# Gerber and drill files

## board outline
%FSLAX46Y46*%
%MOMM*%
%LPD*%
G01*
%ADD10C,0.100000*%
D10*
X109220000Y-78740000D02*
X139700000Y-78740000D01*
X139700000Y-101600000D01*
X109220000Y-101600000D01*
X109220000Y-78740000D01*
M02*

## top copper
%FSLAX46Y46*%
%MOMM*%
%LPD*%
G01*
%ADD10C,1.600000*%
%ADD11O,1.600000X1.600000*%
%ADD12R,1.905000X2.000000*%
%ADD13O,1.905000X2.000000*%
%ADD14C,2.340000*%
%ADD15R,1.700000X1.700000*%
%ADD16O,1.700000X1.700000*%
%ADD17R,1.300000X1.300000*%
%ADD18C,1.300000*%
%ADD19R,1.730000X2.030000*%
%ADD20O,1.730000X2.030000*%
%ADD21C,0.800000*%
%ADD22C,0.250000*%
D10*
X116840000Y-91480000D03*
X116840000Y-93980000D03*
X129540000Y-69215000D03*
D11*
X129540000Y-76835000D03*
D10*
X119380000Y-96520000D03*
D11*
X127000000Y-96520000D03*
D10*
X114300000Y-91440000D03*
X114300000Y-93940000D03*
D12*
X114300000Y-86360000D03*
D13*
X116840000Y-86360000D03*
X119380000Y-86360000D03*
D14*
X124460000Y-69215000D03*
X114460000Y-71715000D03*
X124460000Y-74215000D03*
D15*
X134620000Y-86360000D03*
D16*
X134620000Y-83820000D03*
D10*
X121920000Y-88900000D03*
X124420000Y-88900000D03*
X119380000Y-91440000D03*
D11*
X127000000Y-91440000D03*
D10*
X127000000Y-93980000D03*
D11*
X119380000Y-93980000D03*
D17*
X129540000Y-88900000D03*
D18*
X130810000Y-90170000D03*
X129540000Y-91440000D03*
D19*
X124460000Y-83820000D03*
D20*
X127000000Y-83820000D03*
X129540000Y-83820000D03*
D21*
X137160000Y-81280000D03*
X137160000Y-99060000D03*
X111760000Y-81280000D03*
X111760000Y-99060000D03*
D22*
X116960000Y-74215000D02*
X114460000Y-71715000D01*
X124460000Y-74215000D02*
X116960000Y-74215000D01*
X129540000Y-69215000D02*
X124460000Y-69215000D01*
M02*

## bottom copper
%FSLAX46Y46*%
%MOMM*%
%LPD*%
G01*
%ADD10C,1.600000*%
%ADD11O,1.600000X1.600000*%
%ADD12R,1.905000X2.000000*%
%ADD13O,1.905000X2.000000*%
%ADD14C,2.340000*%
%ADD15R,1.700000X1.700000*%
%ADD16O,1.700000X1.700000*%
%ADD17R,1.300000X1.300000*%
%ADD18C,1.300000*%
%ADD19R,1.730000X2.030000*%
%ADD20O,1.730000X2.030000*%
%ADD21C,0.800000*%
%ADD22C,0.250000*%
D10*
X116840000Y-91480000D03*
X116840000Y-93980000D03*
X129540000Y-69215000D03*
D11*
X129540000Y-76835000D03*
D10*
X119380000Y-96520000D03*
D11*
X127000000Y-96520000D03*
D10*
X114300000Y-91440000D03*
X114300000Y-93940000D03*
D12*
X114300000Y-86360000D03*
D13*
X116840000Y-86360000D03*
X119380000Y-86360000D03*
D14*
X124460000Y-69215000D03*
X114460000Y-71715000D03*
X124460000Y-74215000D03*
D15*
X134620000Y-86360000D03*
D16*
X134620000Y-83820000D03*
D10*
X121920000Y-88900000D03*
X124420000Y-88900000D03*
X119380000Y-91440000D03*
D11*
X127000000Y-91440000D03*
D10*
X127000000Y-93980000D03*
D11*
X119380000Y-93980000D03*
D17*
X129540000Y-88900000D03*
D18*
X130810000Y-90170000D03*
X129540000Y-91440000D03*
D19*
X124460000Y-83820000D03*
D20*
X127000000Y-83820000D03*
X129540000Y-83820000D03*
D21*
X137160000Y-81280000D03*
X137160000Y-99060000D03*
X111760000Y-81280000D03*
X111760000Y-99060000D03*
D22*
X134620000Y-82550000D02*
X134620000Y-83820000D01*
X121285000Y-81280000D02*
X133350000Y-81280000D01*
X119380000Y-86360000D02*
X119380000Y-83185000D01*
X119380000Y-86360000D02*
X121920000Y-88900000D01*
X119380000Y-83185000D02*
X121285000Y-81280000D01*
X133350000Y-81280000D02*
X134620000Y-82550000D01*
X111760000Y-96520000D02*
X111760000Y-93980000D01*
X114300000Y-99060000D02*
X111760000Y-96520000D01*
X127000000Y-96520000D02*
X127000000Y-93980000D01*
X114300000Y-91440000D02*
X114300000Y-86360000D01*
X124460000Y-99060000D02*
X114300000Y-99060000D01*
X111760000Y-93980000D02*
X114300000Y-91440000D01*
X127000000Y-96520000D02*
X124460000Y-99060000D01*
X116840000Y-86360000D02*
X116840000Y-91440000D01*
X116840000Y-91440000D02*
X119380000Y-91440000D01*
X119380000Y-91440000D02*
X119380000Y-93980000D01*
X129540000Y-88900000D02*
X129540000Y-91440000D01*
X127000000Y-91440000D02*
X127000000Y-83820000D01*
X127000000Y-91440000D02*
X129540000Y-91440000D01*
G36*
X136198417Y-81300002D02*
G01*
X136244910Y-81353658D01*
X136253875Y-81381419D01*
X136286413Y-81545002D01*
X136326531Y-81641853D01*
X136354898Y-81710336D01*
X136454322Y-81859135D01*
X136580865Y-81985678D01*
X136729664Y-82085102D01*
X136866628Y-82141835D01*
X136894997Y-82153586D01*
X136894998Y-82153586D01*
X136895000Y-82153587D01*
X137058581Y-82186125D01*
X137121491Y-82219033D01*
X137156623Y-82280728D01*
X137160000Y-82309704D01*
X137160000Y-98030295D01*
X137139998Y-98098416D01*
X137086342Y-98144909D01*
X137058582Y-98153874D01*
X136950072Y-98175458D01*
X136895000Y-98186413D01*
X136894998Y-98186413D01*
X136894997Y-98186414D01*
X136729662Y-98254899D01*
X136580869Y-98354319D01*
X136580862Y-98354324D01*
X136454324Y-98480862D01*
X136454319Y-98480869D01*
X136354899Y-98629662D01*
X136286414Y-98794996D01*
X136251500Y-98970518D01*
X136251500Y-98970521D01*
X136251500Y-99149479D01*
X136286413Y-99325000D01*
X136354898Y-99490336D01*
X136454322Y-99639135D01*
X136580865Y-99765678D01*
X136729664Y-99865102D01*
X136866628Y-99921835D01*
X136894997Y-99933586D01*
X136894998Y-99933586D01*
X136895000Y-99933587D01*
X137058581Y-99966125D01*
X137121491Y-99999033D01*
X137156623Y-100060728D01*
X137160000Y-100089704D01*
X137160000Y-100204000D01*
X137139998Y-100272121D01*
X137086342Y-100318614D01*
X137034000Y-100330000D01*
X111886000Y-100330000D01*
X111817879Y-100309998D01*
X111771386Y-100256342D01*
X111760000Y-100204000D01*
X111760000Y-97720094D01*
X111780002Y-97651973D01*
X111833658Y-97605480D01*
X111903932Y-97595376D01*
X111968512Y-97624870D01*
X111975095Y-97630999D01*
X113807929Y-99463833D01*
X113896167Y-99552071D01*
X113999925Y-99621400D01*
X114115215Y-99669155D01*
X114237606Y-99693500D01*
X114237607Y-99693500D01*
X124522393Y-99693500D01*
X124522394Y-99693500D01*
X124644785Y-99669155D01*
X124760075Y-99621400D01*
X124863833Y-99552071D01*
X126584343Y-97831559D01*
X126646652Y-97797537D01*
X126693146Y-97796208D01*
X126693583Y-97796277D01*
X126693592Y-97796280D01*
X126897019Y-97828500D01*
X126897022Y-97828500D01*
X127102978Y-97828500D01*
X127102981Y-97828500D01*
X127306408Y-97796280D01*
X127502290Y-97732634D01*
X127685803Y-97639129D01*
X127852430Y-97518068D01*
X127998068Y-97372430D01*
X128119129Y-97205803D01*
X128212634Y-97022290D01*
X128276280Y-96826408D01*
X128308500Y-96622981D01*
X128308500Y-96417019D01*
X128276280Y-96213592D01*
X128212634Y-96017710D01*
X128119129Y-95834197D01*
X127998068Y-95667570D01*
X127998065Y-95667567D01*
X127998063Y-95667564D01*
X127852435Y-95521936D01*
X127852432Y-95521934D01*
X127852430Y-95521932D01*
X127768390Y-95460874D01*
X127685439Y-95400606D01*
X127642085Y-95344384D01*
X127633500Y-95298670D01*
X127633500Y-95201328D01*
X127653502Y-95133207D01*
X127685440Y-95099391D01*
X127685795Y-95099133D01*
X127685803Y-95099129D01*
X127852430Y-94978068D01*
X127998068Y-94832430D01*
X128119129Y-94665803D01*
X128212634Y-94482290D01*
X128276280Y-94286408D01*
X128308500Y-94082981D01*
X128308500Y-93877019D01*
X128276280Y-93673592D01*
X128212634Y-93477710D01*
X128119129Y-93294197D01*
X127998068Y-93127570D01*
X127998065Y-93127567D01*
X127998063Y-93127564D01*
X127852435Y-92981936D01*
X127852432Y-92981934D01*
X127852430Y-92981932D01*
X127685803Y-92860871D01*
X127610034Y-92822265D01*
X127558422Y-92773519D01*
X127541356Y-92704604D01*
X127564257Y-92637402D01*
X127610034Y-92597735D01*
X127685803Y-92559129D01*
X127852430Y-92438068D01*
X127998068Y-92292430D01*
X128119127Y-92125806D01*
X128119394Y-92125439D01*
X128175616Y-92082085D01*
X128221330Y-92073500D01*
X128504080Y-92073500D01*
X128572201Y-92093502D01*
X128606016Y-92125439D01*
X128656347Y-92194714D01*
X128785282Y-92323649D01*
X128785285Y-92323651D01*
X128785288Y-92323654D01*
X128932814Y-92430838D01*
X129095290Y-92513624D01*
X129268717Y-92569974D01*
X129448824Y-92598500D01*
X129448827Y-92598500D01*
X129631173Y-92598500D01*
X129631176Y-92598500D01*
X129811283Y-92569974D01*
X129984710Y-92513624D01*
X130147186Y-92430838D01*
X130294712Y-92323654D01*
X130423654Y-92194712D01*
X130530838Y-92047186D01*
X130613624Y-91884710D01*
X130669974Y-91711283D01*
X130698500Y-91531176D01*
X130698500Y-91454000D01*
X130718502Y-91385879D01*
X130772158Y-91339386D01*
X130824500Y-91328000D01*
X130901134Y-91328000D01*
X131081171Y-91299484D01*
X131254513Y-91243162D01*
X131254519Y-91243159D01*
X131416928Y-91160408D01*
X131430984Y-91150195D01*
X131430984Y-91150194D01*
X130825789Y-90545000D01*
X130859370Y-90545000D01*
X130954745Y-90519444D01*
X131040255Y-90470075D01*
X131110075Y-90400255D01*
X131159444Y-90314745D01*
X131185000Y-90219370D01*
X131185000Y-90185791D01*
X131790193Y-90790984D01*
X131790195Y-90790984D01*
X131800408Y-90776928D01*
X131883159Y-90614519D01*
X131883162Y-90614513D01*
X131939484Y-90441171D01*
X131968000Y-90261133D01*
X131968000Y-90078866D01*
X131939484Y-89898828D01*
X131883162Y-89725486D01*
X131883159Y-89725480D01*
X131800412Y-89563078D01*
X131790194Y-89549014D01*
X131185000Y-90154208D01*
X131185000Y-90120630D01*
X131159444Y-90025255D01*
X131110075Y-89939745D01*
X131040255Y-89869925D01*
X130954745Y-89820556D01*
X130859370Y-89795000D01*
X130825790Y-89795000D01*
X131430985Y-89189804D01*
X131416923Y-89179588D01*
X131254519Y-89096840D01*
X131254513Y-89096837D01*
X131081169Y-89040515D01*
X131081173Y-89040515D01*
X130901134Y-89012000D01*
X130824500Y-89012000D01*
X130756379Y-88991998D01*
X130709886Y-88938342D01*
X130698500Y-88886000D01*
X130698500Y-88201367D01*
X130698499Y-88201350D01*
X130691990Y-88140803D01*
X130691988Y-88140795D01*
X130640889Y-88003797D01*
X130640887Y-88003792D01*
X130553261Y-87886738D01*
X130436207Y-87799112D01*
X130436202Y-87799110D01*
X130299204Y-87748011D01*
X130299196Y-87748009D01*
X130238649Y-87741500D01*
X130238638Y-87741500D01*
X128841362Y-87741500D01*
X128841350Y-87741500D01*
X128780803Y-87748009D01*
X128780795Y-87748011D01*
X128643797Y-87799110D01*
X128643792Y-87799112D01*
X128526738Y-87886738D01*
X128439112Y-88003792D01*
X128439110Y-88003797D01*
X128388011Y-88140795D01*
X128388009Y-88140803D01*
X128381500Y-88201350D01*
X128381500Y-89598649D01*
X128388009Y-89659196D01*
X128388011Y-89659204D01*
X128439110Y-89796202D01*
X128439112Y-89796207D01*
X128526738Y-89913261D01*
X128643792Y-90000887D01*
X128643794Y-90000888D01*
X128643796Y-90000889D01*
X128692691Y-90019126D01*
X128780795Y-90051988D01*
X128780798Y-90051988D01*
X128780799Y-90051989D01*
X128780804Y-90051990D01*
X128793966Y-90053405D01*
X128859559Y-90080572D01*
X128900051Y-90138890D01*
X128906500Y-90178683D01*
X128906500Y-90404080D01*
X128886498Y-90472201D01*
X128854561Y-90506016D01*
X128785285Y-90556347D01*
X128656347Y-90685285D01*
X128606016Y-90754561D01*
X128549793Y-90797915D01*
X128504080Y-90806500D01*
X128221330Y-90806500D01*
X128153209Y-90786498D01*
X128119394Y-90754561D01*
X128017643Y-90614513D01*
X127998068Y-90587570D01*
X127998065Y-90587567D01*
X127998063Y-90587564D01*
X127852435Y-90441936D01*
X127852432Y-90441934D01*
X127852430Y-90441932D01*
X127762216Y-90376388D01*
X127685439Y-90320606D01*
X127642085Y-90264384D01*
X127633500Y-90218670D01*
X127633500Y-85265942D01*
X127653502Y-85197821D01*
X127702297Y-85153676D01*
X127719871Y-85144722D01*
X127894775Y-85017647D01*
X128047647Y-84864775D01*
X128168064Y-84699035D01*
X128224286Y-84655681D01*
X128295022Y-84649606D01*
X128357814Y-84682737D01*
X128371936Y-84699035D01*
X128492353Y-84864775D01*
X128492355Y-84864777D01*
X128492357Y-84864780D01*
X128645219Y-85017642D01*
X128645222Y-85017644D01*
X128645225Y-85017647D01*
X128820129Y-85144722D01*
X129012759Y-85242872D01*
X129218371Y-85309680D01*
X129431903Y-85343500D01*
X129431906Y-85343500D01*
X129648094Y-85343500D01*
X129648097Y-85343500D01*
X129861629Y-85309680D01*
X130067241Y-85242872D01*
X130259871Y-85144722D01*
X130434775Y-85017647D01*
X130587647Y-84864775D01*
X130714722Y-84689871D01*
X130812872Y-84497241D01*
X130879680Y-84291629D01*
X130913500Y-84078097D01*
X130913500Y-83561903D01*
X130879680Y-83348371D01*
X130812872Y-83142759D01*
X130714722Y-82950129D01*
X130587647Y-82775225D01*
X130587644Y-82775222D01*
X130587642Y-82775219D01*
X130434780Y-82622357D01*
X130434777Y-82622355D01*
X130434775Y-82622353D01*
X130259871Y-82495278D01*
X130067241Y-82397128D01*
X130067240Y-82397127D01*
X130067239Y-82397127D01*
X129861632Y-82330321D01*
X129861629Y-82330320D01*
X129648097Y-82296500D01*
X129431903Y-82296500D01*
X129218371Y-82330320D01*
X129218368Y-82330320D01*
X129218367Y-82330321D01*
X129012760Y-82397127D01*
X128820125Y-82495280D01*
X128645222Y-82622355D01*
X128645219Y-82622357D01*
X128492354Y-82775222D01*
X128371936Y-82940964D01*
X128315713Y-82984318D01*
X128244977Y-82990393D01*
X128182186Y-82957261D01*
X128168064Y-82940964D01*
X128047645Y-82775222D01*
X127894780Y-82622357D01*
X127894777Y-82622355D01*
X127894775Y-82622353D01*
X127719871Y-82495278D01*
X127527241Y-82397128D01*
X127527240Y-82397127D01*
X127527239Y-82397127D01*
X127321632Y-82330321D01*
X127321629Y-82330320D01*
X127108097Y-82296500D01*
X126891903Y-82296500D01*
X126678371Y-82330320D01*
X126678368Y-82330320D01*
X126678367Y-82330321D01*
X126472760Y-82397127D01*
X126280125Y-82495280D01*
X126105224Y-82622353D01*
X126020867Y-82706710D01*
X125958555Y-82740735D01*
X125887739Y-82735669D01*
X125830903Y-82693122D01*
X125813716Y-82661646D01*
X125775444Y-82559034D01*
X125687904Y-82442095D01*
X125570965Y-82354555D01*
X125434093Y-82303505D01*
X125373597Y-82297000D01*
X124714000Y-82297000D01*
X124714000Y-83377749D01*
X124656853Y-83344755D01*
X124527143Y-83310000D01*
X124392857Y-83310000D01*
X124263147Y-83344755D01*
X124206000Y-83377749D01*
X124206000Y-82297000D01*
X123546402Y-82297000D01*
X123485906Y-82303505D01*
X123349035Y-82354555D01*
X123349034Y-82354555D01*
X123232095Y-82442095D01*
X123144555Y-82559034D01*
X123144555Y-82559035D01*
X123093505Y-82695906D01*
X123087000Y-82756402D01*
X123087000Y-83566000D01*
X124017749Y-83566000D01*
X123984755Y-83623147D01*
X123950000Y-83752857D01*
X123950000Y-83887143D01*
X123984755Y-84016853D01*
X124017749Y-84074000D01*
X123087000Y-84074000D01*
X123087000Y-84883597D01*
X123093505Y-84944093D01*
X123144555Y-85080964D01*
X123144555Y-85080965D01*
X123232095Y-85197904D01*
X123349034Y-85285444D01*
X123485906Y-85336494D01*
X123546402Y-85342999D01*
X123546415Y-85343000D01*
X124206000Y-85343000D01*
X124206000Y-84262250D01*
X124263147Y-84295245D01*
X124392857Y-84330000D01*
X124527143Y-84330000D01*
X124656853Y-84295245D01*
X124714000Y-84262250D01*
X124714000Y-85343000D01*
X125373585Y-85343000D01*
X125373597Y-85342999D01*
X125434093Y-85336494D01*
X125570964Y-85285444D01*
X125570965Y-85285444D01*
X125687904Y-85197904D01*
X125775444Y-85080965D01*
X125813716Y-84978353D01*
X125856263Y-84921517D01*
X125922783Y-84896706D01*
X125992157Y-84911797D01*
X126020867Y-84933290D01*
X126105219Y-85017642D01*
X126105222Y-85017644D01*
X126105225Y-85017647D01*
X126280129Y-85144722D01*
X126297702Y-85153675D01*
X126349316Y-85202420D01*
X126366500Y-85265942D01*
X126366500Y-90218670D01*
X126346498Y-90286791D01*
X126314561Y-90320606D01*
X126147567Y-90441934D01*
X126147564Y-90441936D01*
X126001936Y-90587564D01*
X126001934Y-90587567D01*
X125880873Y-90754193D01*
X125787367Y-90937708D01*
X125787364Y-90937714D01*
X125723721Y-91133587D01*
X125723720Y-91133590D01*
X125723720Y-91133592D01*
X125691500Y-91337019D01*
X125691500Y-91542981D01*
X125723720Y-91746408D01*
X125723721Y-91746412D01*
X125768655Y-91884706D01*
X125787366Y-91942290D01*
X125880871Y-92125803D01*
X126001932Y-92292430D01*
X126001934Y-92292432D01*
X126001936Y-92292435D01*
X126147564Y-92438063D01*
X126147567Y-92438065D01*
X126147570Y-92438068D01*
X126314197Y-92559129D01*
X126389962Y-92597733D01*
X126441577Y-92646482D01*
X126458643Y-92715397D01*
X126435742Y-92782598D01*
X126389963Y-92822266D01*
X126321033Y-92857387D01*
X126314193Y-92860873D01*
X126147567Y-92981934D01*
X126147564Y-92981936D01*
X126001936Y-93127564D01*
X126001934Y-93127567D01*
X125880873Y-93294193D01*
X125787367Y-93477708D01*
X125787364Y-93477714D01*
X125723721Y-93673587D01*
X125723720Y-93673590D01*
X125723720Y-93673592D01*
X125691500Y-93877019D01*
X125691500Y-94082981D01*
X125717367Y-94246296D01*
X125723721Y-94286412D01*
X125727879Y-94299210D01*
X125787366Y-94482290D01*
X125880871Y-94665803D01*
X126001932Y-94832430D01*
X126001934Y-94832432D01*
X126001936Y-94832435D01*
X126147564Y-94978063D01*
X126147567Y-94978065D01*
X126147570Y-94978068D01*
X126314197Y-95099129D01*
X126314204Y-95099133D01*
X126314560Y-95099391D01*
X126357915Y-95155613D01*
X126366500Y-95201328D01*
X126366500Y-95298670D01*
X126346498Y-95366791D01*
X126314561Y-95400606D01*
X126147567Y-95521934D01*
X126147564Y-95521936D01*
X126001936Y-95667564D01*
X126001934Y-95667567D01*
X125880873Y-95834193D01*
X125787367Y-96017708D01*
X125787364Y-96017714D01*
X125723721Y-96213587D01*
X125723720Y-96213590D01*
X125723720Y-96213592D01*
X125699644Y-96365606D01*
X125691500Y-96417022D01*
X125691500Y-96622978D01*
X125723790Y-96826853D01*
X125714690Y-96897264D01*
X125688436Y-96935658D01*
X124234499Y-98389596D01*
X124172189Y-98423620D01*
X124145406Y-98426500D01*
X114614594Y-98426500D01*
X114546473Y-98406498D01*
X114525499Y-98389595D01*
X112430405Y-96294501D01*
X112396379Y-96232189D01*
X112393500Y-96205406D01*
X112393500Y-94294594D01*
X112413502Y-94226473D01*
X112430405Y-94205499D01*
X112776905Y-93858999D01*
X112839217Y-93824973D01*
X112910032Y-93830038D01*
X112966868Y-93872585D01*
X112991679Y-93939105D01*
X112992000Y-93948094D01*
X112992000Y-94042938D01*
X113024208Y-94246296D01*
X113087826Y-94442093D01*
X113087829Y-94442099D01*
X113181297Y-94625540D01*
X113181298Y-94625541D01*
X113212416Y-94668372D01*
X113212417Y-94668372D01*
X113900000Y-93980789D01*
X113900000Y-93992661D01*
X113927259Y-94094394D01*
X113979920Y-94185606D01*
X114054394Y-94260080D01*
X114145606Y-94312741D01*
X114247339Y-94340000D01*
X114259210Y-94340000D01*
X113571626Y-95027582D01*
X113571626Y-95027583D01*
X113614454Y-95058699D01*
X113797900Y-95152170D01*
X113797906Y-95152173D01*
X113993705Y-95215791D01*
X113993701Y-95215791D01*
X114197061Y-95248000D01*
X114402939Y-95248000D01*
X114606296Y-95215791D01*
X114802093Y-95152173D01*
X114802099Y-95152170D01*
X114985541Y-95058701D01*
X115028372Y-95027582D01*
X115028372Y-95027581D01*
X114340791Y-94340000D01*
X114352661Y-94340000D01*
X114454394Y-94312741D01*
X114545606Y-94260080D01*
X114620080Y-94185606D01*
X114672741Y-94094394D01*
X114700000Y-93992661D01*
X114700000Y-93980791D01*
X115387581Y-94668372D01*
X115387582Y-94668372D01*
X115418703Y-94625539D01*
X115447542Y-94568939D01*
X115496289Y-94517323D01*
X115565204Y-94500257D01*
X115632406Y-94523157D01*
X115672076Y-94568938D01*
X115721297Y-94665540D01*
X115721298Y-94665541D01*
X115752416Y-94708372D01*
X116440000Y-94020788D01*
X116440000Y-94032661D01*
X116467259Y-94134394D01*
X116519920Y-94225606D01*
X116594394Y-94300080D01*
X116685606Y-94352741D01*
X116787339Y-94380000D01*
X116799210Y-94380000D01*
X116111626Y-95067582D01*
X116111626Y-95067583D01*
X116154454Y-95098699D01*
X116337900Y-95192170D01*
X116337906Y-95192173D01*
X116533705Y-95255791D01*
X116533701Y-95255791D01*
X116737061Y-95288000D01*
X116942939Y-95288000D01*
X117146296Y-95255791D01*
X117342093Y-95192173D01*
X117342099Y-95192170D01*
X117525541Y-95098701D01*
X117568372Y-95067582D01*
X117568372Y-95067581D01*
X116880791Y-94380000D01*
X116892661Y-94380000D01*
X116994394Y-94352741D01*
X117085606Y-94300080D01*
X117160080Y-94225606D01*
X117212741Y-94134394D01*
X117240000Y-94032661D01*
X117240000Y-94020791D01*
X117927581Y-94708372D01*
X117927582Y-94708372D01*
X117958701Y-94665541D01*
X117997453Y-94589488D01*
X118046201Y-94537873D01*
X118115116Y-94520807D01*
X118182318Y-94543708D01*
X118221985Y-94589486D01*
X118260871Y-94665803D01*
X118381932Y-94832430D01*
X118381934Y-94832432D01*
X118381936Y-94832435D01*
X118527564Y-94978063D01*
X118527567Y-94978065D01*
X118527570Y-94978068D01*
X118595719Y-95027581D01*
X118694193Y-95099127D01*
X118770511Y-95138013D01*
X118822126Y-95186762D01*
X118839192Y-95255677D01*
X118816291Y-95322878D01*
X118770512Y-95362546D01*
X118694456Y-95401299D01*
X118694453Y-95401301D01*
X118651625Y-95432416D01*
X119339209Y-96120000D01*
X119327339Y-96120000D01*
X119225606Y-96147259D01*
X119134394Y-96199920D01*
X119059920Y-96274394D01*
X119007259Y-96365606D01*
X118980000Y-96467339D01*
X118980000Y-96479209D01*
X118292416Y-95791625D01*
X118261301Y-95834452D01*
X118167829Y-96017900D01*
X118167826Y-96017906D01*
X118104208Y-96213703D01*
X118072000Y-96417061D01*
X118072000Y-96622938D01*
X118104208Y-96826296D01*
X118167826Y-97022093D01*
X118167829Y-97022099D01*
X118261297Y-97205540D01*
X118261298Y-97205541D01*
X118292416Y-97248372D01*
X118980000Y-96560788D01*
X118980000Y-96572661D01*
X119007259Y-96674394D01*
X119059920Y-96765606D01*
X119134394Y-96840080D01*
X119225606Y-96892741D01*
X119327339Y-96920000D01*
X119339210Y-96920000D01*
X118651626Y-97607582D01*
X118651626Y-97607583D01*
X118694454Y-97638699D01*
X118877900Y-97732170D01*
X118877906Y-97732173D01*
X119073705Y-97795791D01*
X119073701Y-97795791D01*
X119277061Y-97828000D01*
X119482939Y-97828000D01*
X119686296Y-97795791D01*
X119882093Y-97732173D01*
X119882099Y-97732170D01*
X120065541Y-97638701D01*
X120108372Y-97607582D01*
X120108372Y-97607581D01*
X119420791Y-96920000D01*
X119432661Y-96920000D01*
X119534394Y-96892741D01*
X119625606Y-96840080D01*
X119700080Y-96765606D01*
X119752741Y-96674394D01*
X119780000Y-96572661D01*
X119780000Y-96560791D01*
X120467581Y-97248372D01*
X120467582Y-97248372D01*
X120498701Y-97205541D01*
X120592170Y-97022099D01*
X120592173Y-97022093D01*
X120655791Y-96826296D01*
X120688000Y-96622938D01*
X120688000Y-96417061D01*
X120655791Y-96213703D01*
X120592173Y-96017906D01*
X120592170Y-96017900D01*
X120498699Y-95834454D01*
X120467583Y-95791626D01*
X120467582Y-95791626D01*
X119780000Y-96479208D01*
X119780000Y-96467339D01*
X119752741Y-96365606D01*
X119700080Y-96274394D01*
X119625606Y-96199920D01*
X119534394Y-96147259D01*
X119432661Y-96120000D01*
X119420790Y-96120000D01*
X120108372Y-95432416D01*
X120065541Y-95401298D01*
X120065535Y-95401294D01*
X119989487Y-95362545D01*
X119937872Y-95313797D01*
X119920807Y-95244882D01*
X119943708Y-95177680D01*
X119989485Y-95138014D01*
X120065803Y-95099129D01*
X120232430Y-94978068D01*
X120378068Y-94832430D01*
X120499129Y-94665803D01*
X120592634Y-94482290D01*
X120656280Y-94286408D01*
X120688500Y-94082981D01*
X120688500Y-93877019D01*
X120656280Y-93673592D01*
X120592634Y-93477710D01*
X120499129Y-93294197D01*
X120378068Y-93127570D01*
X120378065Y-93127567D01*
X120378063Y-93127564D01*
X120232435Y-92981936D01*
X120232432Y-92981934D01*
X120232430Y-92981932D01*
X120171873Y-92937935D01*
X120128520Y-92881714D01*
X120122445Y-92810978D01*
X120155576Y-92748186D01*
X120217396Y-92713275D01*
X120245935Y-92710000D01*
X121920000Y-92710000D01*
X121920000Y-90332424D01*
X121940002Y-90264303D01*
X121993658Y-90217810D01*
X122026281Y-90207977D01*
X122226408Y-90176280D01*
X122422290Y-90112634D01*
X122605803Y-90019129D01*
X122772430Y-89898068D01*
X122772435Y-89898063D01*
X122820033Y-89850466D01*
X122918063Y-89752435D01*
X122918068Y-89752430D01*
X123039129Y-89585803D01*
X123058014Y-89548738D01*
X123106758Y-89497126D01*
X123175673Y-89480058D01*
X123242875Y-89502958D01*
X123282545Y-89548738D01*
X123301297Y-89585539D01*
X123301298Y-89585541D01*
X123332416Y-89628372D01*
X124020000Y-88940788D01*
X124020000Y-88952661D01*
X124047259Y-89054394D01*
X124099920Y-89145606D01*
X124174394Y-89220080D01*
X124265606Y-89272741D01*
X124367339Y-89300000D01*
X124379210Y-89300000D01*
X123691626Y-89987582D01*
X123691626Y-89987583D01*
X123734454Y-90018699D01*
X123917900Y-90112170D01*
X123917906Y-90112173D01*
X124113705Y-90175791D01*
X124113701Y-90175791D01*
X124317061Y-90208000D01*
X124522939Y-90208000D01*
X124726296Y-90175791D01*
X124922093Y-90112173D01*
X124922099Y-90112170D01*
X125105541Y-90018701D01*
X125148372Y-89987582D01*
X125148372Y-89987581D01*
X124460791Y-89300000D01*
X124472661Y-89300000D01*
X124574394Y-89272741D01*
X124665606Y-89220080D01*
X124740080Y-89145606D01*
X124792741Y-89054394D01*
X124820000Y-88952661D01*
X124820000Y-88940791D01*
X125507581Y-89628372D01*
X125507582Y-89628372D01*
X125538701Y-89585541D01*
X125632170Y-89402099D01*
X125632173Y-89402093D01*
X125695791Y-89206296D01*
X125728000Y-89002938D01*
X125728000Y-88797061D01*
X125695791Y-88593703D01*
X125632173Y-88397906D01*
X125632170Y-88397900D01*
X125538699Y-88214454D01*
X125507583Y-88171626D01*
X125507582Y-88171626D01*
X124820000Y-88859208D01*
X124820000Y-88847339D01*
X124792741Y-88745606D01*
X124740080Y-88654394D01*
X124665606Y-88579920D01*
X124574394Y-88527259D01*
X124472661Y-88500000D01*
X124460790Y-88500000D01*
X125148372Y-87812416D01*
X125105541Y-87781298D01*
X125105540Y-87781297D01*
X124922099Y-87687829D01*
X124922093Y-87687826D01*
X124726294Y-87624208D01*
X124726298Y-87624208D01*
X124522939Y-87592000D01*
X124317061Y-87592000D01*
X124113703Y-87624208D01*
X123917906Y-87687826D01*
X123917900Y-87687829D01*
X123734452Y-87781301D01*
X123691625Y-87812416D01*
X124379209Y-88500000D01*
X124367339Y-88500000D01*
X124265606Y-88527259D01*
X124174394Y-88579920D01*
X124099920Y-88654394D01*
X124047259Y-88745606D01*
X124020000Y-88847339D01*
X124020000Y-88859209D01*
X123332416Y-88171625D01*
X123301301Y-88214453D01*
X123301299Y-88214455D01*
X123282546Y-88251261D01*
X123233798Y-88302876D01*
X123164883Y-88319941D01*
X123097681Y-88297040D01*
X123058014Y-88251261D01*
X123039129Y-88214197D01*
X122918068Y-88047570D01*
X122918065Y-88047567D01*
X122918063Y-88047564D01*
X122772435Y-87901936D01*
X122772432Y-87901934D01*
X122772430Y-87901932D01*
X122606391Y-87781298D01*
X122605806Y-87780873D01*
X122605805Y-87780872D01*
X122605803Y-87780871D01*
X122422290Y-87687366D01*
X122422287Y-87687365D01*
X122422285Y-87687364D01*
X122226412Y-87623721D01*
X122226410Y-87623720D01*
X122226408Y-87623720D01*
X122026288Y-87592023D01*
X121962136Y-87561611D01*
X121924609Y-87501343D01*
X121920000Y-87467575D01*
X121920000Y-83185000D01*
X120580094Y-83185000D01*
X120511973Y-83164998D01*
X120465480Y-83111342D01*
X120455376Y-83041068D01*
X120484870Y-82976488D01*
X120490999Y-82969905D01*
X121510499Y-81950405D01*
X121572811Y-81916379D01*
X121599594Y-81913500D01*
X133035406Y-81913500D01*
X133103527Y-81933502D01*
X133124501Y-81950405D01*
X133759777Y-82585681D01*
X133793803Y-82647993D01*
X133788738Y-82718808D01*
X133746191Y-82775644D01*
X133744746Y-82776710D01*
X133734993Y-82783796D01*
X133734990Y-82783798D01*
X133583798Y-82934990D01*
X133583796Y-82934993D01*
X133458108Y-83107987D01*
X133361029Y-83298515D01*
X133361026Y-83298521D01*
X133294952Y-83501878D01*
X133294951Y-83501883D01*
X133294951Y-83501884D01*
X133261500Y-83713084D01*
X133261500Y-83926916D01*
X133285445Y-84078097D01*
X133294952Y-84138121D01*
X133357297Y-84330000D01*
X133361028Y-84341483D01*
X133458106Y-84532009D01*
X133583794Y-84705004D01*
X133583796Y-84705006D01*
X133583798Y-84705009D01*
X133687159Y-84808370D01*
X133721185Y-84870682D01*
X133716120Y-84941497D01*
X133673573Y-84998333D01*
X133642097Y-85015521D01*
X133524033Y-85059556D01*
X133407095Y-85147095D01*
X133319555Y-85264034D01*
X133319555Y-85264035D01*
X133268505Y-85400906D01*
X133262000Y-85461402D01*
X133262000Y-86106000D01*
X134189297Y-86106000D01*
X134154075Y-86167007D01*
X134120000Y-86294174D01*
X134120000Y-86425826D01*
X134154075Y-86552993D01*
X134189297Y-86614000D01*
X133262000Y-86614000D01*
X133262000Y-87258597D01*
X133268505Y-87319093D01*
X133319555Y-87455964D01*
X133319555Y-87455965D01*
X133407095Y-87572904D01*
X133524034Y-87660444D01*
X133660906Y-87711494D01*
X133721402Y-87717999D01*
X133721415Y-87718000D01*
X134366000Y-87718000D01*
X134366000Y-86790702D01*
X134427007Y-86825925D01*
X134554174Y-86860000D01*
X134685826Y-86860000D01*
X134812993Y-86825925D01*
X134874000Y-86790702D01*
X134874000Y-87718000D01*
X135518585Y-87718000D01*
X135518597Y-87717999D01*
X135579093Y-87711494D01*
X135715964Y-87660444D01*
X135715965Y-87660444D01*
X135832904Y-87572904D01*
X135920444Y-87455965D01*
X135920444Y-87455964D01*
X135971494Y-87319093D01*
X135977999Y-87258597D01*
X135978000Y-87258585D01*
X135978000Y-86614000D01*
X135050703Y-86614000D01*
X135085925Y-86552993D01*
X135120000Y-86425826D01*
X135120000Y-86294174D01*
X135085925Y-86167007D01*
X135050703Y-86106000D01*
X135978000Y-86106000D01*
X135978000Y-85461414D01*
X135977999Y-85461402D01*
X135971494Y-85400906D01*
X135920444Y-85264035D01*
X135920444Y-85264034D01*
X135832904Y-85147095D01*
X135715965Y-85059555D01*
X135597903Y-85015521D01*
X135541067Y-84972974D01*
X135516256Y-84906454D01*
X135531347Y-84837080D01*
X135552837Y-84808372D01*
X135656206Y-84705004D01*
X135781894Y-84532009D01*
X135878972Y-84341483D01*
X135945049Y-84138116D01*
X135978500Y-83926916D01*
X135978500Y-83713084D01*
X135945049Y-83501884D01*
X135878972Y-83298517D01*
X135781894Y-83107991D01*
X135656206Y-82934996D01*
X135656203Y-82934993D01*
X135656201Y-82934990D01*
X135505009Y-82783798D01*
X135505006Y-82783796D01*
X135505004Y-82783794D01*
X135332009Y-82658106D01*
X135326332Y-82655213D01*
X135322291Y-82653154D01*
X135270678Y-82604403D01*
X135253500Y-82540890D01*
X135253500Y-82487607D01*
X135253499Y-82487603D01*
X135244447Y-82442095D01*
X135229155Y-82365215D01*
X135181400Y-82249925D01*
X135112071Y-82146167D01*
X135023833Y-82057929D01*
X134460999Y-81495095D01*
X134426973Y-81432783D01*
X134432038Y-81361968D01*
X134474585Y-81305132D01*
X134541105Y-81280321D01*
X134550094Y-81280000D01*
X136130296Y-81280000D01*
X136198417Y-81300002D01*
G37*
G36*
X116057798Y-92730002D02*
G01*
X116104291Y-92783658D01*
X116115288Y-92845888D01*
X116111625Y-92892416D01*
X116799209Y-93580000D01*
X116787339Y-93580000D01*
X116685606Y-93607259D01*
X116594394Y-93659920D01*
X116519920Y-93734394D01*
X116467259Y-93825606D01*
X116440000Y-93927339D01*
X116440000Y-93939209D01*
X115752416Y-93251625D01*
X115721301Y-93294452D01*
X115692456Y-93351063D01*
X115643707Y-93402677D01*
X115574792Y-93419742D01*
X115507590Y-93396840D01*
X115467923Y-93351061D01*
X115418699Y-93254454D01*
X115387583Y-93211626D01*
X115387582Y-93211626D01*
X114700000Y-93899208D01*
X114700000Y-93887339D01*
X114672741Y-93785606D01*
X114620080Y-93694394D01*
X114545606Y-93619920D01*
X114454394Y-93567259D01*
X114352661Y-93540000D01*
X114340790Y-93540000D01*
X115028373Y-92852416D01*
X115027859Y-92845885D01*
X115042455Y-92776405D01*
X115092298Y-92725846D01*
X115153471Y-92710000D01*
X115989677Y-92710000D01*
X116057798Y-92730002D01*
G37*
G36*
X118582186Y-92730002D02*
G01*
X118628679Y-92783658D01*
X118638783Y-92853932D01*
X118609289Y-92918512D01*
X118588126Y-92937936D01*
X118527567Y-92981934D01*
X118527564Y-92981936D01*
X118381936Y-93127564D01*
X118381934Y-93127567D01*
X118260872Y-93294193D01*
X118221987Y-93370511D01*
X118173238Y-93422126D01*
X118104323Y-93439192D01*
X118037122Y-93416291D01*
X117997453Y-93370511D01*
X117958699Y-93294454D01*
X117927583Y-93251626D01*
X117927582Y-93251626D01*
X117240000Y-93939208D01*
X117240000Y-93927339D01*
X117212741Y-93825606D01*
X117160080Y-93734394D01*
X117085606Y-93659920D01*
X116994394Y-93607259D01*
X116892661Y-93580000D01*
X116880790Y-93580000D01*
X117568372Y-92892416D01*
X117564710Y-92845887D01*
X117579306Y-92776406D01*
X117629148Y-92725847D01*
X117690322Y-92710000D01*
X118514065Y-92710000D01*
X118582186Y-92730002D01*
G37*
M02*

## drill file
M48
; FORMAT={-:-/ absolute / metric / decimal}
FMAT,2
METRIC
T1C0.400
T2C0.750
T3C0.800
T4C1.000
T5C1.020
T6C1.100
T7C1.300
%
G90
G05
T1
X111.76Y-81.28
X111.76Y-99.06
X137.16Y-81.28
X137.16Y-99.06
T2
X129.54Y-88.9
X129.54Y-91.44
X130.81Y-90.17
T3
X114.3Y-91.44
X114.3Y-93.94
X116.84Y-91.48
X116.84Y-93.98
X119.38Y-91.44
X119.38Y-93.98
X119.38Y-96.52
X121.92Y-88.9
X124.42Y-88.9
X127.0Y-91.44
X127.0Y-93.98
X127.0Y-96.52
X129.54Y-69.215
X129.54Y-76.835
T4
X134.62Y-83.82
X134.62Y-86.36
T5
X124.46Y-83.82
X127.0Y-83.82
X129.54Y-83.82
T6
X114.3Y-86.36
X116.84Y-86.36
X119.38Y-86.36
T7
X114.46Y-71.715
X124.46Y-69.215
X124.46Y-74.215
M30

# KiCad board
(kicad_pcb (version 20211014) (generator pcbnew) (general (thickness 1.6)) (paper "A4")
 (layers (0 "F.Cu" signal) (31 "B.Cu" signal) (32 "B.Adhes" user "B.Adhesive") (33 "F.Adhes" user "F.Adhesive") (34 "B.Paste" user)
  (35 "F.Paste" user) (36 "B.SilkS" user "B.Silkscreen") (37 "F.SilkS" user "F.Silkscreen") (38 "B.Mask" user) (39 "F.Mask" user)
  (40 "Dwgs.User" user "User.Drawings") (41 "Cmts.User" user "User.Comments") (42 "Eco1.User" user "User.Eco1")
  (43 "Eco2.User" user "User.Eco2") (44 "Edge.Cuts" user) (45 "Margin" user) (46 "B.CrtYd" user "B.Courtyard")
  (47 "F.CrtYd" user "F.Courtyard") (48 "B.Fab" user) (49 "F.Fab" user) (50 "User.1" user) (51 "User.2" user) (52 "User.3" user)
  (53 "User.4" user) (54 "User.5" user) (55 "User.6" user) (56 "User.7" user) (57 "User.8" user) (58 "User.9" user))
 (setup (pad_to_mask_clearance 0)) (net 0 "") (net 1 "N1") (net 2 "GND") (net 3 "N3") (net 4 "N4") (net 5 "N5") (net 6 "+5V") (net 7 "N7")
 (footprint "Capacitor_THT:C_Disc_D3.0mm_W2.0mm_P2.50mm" (layer "F.Cu") (at 116.84 91.48 -90)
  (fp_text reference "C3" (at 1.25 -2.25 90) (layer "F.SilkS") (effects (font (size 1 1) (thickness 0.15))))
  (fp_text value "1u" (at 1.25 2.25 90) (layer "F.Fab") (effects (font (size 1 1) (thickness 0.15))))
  (pad "1" thru_hole circle (at 0 0 270) (size 1.6 1.6) (drill 0.8) (layers *.Cu *.Mask) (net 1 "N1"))
  (pad "2" thru_hole circle (at 2.5 0 270) (size 1.6 1.6) (drill 0.8) (layers *.Cu *.Mask) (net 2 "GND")))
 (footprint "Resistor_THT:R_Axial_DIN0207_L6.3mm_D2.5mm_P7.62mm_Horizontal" (layer "F.Cu") (at 129.54 69.215 -90)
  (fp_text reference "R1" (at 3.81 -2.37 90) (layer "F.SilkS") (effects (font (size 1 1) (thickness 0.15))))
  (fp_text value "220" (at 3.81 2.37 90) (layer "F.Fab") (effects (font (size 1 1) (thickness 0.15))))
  (pad "1" thru_hole circle (at 0 0 270) (size 1.6 1.6) (drill 0.8) (layers *.Cu *.Mask) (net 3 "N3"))
  (pad "2" thru_hole oval (at 7.62 0 270) (size 1.6 1.6) (drill 0.8) (layers *.Cu *.Mask) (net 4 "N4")))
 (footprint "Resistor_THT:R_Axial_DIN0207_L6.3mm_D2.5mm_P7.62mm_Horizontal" (layer "F.Cu") (at 119.38 96.52)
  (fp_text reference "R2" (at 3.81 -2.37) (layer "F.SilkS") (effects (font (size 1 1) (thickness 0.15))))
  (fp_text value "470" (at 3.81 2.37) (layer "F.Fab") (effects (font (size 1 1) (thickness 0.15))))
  (pad "1" thru_hole circle (at 0 0) (size 1.6 1.6) (drill 0.8) (layers *.Cu *.Mask) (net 2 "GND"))
  (pad "2" thru_hole oval (at 7.62 0) (size 1.6 1.6) (drill 0.8) (layers *.Cu *.Mask) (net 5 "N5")))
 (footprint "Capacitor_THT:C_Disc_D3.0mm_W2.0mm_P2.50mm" (layer "F.Cu") (at 114.3 91.44 -90)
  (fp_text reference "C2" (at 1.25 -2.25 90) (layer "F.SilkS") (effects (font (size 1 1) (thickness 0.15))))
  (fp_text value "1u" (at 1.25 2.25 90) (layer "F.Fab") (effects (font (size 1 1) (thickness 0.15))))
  (pad "1" thru_hole circle (at 0 0 270) (size 1.6 1.6) (drill 0.8) (layers *.Cu *.Mask) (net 5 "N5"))
  (pad "2" thru_hole circle (at 2.5 0 270) (size 1.6 1.6) (drill 0.8) (layers *.Cu *.Mask) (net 2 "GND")))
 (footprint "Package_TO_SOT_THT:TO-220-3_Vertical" (layer "F.Cu") (at 114.3 86.36) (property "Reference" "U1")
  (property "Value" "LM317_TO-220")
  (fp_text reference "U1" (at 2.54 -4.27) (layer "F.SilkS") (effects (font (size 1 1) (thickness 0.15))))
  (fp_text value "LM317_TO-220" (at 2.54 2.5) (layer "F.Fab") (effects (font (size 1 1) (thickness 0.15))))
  (pad "1" thru_hole rect (at 0 0) (size 1.905 2) (drill 1.1) (layers *.Cu *.Mask) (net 5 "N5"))
  (pad "2" thru_hole oval (at 2.54 0) (size 1.905 2) (drill 1.1) (layers *.Cu *.Mask) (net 1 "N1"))
  (pad "3" thru_hole oval (at 5.08 0) (size 1.905 2) (drill 1.1) (layers *.Cu *.Mask) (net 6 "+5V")))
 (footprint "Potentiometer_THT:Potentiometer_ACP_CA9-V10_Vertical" (layer "F.Cu") (at 124.46 69.215 180) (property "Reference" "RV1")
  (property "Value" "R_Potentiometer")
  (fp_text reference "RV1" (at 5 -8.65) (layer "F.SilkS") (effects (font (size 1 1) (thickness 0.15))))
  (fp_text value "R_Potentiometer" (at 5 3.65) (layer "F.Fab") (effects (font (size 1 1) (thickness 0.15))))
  (pad "1" thru_hole circle (at 0 0 180) (size 2.34 2.34) (drill 1.3) (layers *.Cu *.Mask) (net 3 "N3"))
  (pad "2" thru_hole circle (at 10 -2.5 180) (size 2.34 2.34) (drill 1.3) (layers *.Cu *.Mask) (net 2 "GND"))
  (pad "3" thru_hole circle (at 0 -5 180) (size 2.34 2.34) (drill 1.3) (layers *.Cu *.Mask) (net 2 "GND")))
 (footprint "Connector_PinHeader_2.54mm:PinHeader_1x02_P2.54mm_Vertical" (layer "F.Cu") (at 134.62 86.36 180) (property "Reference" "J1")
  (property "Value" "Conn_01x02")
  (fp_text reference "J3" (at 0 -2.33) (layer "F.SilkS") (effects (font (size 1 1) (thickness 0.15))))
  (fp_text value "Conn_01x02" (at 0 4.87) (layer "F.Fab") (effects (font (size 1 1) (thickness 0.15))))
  (pad "1" thru_hole rect (at 0 0 180) (size 1.7 1.7) (drill 1) (layers *.Cu *.Mask) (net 2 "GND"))
  (pad "2" thru_hole oval (at 0 2.54 180) (size 1.7 1.7) (drill 1) (layers *.Cu *.Mask) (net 6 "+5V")))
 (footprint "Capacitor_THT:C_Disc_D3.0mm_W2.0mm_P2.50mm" (layer "F.Cu") (at 121.92 88.9) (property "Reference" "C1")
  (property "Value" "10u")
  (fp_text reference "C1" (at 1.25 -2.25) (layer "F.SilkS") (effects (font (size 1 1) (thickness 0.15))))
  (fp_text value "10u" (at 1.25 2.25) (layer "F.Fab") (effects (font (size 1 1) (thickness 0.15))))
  (pad "1" thru_hole circle (at 0 0) (size 1.6 1.6) (drill 0.8) (layers *.Cu *.Mask) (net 6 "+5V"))
  (pad "2" thru_hole circle (at 2.5 0) (size 1.6 1.6) (drill 0.8) (layers *.Cu *.Mask) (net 2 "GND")))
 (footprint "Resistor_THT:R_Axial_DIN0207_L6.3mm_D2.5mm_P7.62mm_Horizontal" (layer "F.Cu") (at 119.38 91.44)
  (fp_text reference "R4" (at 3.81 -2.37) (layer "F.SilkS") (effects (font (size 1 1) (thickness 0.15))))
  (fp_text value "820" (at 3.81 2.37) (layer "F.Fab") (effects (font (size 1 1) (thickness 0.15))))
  (pad "1" thru_hole circle (at 0 0) (size 1.6 1.6) (drill 0.8) (layers *.Cu *.Mask) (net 1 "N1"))
  (pad "2" thru_hole oval (at 7.62 0) (size 1.6 1.6) (drill 0.8) (layers *.Cu *.Mask) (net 4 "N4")))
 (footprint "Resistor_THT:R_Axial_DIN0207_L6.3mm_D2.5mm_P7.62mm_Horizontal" (layer "F.Cu") (at 127 93.98 180) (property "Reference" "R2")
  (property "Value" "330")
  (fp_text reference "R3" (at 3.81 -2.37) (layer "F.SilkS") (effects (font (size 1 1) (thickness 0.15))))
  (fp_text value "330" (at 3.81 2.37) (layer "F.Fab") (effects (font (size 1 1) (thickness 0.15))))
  (pad "1" thru_hole circle (at 0 0 180) (size 1.6 1.6) (drill 0.8) (layers *.Cu *.Mask) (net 5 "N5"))
  (pad "2" thru_hole oval (at 7.62 0 180) (size 1.6 1.6) (drill 0.8) (layers *.Cu *.Mask) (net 1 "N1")))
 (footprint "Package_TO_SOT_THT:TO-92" (layer "F.Cu") (at 129.54 88.9 -90) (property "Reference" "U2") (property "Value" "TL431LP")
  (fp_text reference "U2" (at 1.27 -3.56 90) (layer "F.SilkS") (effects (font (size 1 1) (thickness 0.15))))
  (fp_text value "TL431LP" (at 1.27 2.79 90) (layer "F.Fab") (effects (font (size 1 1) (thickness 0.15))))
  (pad "1" thru_hole rect (at 0 0 270) (size 1.3 1.3) (drill 0.75) (layers *.Cu *.Mask) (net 4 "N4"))
  (pad "2" thru_hole circle (at 1.27 -1.27 270) (size 1.3 1.3) (drill 0.75) (layers *.Cu *.Mask) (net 2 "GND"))
  (pad "3" thru_hole circle (at 2.54 0 270) (size 1.3 1.3) (drill 0.75) (layers *.Cu *.Mask) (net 4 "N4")))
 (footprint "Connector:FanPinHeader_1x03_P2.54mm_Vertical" (layer "F.Cu") (at 124.46 83.82) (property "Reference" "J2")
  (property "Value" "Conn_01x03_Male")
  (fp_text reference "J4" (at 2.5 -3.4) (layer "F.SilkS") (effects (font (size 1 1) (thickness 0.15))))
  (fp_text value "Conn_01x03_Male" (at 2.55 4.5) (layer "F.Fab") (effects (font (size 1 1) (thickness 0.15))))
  (pad "1" thru_hole rect (at 0 0 90) (size 2.03 1.73) (drill 1.02) (layers *.Cu *.Mask) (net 2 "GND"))
  (pad "2" thru_hole oval (at 2.54 0 90) (size 2.03 1.73) (drill 1.02) (layers *.Cu *.Mask) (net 4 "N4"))
  (pad "3" thru_hole oval (at 5.08 0 90) (size 2.03 1.73) (drill 1.02) (layers *.Cu *.Mask) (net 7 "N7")))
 (gr_rect (start 109.22 78.74) (end 139.7 101.6) (layer "Edge.Cuts") (width 0.1) (fill none))
 (via (at 137.16 81.28) (size 0.8) (drill 0.4) (layers "F.Cu" "B.Cu") (free) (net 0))
 (via (at 137.16 99.06) (size 0.8) (drill 0.4) (layers "F.Cu" "B.Cu") (free) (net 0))
 (via (at 111.76 81.28) (size 0.8) (drill 0.4) (layers "F.Cu" "B.Cu") (free) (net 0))
 (segment (start 134.62 82.55) (end 134.62 83.82) (width 0.25) (layer "B.Cu") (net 6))
 (segment (start 121.285 81.28) (end 133.35 81.28) (width 0.25) (layer "B.Cu") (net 6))
 (segment (start 119.38 86.36) (end 119.38 83.185) (width 0.25) (layer "B.Cu") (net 6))
 (segment (start 119.38 86.36) (end 121.92 88.9) (width 0.25) (layer "B.Cu") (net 6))
 (segment (start 119.38 83.185) (end 121.285 81.28) (width 0.25) (layer "B.Cu") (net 6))
 (segment (start 133.35 81.28) (end 134.62 82.55) (width 0.25) (layer "B.Cu") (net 6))
 (segment (start 116.96 74.215) (end 114.46 71.715) (width 0.25) (layer "F.Cu") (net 2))
 (segment (start 124.46 74.215) (end 116.96 74.215) (width 0.25) (layer "F.Cu") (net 2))
 (via (at 111.76 99.06) (size 0.8) (drill 0.4) (layers "F.Cu" "B.Cu") (free) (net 2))
 (segment (start 111.76 96.52) (end 111.76 93.98) (width 0.25) (layer "B.Cu") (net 5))
 (segment (start 114.3 99.06) (end 111.76 96.52) (width 0.25) (layer "B.Cu") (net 5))
 (segment (start 127 96.52) (end 127 93.98) (width 0.25) (layer "B.Cu") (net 5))
 (segment (start 114.3 91.44) (end 114.3 86.36) (width 0.25) (layer "B.Cu") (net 5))
 (segment (start 124.46 99.06) (end 114.3 99.06) (width 0.25) (layer "B.Cu") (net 5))
 (segment (start 111.76 93.98) (end 114.3 91.44) (width 0.25) (layer "B.Cu") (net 5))
 (segment (start 127 96.52) (end 124.46 99.06) (width 0.25) (layer "B.Cu") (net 5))
 (segment (start 116.84 86.36) (end 116.84 91.44) (width 0.25) (layer "B.Cu") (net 1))
 (segment (start 116.84 91.44) (end 119.38 91.44) (width 0.25) (layer "B.Cu") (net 1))
 (segment (start 119.38 91.44) (end 119.38 93.98) (width 0.25) (layer "B.Cu") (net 1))
 (segment (start 129.54 88.9) (end 129.54 91.44) (width 0.25) (layer "B.Cu") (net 4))
 (segment (start 127 91.44) (end 127 83.82) (width 0.25) (layer "B.Cu") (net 4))
 (segment (start 127 91.44) (end 129.54 91.44) (width 0.25) (layer "B.Cu") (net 4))
 (segment (start 129.54 69.215) (end 124.46 69.215) (width 0.25) (layer "F.Cu") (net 3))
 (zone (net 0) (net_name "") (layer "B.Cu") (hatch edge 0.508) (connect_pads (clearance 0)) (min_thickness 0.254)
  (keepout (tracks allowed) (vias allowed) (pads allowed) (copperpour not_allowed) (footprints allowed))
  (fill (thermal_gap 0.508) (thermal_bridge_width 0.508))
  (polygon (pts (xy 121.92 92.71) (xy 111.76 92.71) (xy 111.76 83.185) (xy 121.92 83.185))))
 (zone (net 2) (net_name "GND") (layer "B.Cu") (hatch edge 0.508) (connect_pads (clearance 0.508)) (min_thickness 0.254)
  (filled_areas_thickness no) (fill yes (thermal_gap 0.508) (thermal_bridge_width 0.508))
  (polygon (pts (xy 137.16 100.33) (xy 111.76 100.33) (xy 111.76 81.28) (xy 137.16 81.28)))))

